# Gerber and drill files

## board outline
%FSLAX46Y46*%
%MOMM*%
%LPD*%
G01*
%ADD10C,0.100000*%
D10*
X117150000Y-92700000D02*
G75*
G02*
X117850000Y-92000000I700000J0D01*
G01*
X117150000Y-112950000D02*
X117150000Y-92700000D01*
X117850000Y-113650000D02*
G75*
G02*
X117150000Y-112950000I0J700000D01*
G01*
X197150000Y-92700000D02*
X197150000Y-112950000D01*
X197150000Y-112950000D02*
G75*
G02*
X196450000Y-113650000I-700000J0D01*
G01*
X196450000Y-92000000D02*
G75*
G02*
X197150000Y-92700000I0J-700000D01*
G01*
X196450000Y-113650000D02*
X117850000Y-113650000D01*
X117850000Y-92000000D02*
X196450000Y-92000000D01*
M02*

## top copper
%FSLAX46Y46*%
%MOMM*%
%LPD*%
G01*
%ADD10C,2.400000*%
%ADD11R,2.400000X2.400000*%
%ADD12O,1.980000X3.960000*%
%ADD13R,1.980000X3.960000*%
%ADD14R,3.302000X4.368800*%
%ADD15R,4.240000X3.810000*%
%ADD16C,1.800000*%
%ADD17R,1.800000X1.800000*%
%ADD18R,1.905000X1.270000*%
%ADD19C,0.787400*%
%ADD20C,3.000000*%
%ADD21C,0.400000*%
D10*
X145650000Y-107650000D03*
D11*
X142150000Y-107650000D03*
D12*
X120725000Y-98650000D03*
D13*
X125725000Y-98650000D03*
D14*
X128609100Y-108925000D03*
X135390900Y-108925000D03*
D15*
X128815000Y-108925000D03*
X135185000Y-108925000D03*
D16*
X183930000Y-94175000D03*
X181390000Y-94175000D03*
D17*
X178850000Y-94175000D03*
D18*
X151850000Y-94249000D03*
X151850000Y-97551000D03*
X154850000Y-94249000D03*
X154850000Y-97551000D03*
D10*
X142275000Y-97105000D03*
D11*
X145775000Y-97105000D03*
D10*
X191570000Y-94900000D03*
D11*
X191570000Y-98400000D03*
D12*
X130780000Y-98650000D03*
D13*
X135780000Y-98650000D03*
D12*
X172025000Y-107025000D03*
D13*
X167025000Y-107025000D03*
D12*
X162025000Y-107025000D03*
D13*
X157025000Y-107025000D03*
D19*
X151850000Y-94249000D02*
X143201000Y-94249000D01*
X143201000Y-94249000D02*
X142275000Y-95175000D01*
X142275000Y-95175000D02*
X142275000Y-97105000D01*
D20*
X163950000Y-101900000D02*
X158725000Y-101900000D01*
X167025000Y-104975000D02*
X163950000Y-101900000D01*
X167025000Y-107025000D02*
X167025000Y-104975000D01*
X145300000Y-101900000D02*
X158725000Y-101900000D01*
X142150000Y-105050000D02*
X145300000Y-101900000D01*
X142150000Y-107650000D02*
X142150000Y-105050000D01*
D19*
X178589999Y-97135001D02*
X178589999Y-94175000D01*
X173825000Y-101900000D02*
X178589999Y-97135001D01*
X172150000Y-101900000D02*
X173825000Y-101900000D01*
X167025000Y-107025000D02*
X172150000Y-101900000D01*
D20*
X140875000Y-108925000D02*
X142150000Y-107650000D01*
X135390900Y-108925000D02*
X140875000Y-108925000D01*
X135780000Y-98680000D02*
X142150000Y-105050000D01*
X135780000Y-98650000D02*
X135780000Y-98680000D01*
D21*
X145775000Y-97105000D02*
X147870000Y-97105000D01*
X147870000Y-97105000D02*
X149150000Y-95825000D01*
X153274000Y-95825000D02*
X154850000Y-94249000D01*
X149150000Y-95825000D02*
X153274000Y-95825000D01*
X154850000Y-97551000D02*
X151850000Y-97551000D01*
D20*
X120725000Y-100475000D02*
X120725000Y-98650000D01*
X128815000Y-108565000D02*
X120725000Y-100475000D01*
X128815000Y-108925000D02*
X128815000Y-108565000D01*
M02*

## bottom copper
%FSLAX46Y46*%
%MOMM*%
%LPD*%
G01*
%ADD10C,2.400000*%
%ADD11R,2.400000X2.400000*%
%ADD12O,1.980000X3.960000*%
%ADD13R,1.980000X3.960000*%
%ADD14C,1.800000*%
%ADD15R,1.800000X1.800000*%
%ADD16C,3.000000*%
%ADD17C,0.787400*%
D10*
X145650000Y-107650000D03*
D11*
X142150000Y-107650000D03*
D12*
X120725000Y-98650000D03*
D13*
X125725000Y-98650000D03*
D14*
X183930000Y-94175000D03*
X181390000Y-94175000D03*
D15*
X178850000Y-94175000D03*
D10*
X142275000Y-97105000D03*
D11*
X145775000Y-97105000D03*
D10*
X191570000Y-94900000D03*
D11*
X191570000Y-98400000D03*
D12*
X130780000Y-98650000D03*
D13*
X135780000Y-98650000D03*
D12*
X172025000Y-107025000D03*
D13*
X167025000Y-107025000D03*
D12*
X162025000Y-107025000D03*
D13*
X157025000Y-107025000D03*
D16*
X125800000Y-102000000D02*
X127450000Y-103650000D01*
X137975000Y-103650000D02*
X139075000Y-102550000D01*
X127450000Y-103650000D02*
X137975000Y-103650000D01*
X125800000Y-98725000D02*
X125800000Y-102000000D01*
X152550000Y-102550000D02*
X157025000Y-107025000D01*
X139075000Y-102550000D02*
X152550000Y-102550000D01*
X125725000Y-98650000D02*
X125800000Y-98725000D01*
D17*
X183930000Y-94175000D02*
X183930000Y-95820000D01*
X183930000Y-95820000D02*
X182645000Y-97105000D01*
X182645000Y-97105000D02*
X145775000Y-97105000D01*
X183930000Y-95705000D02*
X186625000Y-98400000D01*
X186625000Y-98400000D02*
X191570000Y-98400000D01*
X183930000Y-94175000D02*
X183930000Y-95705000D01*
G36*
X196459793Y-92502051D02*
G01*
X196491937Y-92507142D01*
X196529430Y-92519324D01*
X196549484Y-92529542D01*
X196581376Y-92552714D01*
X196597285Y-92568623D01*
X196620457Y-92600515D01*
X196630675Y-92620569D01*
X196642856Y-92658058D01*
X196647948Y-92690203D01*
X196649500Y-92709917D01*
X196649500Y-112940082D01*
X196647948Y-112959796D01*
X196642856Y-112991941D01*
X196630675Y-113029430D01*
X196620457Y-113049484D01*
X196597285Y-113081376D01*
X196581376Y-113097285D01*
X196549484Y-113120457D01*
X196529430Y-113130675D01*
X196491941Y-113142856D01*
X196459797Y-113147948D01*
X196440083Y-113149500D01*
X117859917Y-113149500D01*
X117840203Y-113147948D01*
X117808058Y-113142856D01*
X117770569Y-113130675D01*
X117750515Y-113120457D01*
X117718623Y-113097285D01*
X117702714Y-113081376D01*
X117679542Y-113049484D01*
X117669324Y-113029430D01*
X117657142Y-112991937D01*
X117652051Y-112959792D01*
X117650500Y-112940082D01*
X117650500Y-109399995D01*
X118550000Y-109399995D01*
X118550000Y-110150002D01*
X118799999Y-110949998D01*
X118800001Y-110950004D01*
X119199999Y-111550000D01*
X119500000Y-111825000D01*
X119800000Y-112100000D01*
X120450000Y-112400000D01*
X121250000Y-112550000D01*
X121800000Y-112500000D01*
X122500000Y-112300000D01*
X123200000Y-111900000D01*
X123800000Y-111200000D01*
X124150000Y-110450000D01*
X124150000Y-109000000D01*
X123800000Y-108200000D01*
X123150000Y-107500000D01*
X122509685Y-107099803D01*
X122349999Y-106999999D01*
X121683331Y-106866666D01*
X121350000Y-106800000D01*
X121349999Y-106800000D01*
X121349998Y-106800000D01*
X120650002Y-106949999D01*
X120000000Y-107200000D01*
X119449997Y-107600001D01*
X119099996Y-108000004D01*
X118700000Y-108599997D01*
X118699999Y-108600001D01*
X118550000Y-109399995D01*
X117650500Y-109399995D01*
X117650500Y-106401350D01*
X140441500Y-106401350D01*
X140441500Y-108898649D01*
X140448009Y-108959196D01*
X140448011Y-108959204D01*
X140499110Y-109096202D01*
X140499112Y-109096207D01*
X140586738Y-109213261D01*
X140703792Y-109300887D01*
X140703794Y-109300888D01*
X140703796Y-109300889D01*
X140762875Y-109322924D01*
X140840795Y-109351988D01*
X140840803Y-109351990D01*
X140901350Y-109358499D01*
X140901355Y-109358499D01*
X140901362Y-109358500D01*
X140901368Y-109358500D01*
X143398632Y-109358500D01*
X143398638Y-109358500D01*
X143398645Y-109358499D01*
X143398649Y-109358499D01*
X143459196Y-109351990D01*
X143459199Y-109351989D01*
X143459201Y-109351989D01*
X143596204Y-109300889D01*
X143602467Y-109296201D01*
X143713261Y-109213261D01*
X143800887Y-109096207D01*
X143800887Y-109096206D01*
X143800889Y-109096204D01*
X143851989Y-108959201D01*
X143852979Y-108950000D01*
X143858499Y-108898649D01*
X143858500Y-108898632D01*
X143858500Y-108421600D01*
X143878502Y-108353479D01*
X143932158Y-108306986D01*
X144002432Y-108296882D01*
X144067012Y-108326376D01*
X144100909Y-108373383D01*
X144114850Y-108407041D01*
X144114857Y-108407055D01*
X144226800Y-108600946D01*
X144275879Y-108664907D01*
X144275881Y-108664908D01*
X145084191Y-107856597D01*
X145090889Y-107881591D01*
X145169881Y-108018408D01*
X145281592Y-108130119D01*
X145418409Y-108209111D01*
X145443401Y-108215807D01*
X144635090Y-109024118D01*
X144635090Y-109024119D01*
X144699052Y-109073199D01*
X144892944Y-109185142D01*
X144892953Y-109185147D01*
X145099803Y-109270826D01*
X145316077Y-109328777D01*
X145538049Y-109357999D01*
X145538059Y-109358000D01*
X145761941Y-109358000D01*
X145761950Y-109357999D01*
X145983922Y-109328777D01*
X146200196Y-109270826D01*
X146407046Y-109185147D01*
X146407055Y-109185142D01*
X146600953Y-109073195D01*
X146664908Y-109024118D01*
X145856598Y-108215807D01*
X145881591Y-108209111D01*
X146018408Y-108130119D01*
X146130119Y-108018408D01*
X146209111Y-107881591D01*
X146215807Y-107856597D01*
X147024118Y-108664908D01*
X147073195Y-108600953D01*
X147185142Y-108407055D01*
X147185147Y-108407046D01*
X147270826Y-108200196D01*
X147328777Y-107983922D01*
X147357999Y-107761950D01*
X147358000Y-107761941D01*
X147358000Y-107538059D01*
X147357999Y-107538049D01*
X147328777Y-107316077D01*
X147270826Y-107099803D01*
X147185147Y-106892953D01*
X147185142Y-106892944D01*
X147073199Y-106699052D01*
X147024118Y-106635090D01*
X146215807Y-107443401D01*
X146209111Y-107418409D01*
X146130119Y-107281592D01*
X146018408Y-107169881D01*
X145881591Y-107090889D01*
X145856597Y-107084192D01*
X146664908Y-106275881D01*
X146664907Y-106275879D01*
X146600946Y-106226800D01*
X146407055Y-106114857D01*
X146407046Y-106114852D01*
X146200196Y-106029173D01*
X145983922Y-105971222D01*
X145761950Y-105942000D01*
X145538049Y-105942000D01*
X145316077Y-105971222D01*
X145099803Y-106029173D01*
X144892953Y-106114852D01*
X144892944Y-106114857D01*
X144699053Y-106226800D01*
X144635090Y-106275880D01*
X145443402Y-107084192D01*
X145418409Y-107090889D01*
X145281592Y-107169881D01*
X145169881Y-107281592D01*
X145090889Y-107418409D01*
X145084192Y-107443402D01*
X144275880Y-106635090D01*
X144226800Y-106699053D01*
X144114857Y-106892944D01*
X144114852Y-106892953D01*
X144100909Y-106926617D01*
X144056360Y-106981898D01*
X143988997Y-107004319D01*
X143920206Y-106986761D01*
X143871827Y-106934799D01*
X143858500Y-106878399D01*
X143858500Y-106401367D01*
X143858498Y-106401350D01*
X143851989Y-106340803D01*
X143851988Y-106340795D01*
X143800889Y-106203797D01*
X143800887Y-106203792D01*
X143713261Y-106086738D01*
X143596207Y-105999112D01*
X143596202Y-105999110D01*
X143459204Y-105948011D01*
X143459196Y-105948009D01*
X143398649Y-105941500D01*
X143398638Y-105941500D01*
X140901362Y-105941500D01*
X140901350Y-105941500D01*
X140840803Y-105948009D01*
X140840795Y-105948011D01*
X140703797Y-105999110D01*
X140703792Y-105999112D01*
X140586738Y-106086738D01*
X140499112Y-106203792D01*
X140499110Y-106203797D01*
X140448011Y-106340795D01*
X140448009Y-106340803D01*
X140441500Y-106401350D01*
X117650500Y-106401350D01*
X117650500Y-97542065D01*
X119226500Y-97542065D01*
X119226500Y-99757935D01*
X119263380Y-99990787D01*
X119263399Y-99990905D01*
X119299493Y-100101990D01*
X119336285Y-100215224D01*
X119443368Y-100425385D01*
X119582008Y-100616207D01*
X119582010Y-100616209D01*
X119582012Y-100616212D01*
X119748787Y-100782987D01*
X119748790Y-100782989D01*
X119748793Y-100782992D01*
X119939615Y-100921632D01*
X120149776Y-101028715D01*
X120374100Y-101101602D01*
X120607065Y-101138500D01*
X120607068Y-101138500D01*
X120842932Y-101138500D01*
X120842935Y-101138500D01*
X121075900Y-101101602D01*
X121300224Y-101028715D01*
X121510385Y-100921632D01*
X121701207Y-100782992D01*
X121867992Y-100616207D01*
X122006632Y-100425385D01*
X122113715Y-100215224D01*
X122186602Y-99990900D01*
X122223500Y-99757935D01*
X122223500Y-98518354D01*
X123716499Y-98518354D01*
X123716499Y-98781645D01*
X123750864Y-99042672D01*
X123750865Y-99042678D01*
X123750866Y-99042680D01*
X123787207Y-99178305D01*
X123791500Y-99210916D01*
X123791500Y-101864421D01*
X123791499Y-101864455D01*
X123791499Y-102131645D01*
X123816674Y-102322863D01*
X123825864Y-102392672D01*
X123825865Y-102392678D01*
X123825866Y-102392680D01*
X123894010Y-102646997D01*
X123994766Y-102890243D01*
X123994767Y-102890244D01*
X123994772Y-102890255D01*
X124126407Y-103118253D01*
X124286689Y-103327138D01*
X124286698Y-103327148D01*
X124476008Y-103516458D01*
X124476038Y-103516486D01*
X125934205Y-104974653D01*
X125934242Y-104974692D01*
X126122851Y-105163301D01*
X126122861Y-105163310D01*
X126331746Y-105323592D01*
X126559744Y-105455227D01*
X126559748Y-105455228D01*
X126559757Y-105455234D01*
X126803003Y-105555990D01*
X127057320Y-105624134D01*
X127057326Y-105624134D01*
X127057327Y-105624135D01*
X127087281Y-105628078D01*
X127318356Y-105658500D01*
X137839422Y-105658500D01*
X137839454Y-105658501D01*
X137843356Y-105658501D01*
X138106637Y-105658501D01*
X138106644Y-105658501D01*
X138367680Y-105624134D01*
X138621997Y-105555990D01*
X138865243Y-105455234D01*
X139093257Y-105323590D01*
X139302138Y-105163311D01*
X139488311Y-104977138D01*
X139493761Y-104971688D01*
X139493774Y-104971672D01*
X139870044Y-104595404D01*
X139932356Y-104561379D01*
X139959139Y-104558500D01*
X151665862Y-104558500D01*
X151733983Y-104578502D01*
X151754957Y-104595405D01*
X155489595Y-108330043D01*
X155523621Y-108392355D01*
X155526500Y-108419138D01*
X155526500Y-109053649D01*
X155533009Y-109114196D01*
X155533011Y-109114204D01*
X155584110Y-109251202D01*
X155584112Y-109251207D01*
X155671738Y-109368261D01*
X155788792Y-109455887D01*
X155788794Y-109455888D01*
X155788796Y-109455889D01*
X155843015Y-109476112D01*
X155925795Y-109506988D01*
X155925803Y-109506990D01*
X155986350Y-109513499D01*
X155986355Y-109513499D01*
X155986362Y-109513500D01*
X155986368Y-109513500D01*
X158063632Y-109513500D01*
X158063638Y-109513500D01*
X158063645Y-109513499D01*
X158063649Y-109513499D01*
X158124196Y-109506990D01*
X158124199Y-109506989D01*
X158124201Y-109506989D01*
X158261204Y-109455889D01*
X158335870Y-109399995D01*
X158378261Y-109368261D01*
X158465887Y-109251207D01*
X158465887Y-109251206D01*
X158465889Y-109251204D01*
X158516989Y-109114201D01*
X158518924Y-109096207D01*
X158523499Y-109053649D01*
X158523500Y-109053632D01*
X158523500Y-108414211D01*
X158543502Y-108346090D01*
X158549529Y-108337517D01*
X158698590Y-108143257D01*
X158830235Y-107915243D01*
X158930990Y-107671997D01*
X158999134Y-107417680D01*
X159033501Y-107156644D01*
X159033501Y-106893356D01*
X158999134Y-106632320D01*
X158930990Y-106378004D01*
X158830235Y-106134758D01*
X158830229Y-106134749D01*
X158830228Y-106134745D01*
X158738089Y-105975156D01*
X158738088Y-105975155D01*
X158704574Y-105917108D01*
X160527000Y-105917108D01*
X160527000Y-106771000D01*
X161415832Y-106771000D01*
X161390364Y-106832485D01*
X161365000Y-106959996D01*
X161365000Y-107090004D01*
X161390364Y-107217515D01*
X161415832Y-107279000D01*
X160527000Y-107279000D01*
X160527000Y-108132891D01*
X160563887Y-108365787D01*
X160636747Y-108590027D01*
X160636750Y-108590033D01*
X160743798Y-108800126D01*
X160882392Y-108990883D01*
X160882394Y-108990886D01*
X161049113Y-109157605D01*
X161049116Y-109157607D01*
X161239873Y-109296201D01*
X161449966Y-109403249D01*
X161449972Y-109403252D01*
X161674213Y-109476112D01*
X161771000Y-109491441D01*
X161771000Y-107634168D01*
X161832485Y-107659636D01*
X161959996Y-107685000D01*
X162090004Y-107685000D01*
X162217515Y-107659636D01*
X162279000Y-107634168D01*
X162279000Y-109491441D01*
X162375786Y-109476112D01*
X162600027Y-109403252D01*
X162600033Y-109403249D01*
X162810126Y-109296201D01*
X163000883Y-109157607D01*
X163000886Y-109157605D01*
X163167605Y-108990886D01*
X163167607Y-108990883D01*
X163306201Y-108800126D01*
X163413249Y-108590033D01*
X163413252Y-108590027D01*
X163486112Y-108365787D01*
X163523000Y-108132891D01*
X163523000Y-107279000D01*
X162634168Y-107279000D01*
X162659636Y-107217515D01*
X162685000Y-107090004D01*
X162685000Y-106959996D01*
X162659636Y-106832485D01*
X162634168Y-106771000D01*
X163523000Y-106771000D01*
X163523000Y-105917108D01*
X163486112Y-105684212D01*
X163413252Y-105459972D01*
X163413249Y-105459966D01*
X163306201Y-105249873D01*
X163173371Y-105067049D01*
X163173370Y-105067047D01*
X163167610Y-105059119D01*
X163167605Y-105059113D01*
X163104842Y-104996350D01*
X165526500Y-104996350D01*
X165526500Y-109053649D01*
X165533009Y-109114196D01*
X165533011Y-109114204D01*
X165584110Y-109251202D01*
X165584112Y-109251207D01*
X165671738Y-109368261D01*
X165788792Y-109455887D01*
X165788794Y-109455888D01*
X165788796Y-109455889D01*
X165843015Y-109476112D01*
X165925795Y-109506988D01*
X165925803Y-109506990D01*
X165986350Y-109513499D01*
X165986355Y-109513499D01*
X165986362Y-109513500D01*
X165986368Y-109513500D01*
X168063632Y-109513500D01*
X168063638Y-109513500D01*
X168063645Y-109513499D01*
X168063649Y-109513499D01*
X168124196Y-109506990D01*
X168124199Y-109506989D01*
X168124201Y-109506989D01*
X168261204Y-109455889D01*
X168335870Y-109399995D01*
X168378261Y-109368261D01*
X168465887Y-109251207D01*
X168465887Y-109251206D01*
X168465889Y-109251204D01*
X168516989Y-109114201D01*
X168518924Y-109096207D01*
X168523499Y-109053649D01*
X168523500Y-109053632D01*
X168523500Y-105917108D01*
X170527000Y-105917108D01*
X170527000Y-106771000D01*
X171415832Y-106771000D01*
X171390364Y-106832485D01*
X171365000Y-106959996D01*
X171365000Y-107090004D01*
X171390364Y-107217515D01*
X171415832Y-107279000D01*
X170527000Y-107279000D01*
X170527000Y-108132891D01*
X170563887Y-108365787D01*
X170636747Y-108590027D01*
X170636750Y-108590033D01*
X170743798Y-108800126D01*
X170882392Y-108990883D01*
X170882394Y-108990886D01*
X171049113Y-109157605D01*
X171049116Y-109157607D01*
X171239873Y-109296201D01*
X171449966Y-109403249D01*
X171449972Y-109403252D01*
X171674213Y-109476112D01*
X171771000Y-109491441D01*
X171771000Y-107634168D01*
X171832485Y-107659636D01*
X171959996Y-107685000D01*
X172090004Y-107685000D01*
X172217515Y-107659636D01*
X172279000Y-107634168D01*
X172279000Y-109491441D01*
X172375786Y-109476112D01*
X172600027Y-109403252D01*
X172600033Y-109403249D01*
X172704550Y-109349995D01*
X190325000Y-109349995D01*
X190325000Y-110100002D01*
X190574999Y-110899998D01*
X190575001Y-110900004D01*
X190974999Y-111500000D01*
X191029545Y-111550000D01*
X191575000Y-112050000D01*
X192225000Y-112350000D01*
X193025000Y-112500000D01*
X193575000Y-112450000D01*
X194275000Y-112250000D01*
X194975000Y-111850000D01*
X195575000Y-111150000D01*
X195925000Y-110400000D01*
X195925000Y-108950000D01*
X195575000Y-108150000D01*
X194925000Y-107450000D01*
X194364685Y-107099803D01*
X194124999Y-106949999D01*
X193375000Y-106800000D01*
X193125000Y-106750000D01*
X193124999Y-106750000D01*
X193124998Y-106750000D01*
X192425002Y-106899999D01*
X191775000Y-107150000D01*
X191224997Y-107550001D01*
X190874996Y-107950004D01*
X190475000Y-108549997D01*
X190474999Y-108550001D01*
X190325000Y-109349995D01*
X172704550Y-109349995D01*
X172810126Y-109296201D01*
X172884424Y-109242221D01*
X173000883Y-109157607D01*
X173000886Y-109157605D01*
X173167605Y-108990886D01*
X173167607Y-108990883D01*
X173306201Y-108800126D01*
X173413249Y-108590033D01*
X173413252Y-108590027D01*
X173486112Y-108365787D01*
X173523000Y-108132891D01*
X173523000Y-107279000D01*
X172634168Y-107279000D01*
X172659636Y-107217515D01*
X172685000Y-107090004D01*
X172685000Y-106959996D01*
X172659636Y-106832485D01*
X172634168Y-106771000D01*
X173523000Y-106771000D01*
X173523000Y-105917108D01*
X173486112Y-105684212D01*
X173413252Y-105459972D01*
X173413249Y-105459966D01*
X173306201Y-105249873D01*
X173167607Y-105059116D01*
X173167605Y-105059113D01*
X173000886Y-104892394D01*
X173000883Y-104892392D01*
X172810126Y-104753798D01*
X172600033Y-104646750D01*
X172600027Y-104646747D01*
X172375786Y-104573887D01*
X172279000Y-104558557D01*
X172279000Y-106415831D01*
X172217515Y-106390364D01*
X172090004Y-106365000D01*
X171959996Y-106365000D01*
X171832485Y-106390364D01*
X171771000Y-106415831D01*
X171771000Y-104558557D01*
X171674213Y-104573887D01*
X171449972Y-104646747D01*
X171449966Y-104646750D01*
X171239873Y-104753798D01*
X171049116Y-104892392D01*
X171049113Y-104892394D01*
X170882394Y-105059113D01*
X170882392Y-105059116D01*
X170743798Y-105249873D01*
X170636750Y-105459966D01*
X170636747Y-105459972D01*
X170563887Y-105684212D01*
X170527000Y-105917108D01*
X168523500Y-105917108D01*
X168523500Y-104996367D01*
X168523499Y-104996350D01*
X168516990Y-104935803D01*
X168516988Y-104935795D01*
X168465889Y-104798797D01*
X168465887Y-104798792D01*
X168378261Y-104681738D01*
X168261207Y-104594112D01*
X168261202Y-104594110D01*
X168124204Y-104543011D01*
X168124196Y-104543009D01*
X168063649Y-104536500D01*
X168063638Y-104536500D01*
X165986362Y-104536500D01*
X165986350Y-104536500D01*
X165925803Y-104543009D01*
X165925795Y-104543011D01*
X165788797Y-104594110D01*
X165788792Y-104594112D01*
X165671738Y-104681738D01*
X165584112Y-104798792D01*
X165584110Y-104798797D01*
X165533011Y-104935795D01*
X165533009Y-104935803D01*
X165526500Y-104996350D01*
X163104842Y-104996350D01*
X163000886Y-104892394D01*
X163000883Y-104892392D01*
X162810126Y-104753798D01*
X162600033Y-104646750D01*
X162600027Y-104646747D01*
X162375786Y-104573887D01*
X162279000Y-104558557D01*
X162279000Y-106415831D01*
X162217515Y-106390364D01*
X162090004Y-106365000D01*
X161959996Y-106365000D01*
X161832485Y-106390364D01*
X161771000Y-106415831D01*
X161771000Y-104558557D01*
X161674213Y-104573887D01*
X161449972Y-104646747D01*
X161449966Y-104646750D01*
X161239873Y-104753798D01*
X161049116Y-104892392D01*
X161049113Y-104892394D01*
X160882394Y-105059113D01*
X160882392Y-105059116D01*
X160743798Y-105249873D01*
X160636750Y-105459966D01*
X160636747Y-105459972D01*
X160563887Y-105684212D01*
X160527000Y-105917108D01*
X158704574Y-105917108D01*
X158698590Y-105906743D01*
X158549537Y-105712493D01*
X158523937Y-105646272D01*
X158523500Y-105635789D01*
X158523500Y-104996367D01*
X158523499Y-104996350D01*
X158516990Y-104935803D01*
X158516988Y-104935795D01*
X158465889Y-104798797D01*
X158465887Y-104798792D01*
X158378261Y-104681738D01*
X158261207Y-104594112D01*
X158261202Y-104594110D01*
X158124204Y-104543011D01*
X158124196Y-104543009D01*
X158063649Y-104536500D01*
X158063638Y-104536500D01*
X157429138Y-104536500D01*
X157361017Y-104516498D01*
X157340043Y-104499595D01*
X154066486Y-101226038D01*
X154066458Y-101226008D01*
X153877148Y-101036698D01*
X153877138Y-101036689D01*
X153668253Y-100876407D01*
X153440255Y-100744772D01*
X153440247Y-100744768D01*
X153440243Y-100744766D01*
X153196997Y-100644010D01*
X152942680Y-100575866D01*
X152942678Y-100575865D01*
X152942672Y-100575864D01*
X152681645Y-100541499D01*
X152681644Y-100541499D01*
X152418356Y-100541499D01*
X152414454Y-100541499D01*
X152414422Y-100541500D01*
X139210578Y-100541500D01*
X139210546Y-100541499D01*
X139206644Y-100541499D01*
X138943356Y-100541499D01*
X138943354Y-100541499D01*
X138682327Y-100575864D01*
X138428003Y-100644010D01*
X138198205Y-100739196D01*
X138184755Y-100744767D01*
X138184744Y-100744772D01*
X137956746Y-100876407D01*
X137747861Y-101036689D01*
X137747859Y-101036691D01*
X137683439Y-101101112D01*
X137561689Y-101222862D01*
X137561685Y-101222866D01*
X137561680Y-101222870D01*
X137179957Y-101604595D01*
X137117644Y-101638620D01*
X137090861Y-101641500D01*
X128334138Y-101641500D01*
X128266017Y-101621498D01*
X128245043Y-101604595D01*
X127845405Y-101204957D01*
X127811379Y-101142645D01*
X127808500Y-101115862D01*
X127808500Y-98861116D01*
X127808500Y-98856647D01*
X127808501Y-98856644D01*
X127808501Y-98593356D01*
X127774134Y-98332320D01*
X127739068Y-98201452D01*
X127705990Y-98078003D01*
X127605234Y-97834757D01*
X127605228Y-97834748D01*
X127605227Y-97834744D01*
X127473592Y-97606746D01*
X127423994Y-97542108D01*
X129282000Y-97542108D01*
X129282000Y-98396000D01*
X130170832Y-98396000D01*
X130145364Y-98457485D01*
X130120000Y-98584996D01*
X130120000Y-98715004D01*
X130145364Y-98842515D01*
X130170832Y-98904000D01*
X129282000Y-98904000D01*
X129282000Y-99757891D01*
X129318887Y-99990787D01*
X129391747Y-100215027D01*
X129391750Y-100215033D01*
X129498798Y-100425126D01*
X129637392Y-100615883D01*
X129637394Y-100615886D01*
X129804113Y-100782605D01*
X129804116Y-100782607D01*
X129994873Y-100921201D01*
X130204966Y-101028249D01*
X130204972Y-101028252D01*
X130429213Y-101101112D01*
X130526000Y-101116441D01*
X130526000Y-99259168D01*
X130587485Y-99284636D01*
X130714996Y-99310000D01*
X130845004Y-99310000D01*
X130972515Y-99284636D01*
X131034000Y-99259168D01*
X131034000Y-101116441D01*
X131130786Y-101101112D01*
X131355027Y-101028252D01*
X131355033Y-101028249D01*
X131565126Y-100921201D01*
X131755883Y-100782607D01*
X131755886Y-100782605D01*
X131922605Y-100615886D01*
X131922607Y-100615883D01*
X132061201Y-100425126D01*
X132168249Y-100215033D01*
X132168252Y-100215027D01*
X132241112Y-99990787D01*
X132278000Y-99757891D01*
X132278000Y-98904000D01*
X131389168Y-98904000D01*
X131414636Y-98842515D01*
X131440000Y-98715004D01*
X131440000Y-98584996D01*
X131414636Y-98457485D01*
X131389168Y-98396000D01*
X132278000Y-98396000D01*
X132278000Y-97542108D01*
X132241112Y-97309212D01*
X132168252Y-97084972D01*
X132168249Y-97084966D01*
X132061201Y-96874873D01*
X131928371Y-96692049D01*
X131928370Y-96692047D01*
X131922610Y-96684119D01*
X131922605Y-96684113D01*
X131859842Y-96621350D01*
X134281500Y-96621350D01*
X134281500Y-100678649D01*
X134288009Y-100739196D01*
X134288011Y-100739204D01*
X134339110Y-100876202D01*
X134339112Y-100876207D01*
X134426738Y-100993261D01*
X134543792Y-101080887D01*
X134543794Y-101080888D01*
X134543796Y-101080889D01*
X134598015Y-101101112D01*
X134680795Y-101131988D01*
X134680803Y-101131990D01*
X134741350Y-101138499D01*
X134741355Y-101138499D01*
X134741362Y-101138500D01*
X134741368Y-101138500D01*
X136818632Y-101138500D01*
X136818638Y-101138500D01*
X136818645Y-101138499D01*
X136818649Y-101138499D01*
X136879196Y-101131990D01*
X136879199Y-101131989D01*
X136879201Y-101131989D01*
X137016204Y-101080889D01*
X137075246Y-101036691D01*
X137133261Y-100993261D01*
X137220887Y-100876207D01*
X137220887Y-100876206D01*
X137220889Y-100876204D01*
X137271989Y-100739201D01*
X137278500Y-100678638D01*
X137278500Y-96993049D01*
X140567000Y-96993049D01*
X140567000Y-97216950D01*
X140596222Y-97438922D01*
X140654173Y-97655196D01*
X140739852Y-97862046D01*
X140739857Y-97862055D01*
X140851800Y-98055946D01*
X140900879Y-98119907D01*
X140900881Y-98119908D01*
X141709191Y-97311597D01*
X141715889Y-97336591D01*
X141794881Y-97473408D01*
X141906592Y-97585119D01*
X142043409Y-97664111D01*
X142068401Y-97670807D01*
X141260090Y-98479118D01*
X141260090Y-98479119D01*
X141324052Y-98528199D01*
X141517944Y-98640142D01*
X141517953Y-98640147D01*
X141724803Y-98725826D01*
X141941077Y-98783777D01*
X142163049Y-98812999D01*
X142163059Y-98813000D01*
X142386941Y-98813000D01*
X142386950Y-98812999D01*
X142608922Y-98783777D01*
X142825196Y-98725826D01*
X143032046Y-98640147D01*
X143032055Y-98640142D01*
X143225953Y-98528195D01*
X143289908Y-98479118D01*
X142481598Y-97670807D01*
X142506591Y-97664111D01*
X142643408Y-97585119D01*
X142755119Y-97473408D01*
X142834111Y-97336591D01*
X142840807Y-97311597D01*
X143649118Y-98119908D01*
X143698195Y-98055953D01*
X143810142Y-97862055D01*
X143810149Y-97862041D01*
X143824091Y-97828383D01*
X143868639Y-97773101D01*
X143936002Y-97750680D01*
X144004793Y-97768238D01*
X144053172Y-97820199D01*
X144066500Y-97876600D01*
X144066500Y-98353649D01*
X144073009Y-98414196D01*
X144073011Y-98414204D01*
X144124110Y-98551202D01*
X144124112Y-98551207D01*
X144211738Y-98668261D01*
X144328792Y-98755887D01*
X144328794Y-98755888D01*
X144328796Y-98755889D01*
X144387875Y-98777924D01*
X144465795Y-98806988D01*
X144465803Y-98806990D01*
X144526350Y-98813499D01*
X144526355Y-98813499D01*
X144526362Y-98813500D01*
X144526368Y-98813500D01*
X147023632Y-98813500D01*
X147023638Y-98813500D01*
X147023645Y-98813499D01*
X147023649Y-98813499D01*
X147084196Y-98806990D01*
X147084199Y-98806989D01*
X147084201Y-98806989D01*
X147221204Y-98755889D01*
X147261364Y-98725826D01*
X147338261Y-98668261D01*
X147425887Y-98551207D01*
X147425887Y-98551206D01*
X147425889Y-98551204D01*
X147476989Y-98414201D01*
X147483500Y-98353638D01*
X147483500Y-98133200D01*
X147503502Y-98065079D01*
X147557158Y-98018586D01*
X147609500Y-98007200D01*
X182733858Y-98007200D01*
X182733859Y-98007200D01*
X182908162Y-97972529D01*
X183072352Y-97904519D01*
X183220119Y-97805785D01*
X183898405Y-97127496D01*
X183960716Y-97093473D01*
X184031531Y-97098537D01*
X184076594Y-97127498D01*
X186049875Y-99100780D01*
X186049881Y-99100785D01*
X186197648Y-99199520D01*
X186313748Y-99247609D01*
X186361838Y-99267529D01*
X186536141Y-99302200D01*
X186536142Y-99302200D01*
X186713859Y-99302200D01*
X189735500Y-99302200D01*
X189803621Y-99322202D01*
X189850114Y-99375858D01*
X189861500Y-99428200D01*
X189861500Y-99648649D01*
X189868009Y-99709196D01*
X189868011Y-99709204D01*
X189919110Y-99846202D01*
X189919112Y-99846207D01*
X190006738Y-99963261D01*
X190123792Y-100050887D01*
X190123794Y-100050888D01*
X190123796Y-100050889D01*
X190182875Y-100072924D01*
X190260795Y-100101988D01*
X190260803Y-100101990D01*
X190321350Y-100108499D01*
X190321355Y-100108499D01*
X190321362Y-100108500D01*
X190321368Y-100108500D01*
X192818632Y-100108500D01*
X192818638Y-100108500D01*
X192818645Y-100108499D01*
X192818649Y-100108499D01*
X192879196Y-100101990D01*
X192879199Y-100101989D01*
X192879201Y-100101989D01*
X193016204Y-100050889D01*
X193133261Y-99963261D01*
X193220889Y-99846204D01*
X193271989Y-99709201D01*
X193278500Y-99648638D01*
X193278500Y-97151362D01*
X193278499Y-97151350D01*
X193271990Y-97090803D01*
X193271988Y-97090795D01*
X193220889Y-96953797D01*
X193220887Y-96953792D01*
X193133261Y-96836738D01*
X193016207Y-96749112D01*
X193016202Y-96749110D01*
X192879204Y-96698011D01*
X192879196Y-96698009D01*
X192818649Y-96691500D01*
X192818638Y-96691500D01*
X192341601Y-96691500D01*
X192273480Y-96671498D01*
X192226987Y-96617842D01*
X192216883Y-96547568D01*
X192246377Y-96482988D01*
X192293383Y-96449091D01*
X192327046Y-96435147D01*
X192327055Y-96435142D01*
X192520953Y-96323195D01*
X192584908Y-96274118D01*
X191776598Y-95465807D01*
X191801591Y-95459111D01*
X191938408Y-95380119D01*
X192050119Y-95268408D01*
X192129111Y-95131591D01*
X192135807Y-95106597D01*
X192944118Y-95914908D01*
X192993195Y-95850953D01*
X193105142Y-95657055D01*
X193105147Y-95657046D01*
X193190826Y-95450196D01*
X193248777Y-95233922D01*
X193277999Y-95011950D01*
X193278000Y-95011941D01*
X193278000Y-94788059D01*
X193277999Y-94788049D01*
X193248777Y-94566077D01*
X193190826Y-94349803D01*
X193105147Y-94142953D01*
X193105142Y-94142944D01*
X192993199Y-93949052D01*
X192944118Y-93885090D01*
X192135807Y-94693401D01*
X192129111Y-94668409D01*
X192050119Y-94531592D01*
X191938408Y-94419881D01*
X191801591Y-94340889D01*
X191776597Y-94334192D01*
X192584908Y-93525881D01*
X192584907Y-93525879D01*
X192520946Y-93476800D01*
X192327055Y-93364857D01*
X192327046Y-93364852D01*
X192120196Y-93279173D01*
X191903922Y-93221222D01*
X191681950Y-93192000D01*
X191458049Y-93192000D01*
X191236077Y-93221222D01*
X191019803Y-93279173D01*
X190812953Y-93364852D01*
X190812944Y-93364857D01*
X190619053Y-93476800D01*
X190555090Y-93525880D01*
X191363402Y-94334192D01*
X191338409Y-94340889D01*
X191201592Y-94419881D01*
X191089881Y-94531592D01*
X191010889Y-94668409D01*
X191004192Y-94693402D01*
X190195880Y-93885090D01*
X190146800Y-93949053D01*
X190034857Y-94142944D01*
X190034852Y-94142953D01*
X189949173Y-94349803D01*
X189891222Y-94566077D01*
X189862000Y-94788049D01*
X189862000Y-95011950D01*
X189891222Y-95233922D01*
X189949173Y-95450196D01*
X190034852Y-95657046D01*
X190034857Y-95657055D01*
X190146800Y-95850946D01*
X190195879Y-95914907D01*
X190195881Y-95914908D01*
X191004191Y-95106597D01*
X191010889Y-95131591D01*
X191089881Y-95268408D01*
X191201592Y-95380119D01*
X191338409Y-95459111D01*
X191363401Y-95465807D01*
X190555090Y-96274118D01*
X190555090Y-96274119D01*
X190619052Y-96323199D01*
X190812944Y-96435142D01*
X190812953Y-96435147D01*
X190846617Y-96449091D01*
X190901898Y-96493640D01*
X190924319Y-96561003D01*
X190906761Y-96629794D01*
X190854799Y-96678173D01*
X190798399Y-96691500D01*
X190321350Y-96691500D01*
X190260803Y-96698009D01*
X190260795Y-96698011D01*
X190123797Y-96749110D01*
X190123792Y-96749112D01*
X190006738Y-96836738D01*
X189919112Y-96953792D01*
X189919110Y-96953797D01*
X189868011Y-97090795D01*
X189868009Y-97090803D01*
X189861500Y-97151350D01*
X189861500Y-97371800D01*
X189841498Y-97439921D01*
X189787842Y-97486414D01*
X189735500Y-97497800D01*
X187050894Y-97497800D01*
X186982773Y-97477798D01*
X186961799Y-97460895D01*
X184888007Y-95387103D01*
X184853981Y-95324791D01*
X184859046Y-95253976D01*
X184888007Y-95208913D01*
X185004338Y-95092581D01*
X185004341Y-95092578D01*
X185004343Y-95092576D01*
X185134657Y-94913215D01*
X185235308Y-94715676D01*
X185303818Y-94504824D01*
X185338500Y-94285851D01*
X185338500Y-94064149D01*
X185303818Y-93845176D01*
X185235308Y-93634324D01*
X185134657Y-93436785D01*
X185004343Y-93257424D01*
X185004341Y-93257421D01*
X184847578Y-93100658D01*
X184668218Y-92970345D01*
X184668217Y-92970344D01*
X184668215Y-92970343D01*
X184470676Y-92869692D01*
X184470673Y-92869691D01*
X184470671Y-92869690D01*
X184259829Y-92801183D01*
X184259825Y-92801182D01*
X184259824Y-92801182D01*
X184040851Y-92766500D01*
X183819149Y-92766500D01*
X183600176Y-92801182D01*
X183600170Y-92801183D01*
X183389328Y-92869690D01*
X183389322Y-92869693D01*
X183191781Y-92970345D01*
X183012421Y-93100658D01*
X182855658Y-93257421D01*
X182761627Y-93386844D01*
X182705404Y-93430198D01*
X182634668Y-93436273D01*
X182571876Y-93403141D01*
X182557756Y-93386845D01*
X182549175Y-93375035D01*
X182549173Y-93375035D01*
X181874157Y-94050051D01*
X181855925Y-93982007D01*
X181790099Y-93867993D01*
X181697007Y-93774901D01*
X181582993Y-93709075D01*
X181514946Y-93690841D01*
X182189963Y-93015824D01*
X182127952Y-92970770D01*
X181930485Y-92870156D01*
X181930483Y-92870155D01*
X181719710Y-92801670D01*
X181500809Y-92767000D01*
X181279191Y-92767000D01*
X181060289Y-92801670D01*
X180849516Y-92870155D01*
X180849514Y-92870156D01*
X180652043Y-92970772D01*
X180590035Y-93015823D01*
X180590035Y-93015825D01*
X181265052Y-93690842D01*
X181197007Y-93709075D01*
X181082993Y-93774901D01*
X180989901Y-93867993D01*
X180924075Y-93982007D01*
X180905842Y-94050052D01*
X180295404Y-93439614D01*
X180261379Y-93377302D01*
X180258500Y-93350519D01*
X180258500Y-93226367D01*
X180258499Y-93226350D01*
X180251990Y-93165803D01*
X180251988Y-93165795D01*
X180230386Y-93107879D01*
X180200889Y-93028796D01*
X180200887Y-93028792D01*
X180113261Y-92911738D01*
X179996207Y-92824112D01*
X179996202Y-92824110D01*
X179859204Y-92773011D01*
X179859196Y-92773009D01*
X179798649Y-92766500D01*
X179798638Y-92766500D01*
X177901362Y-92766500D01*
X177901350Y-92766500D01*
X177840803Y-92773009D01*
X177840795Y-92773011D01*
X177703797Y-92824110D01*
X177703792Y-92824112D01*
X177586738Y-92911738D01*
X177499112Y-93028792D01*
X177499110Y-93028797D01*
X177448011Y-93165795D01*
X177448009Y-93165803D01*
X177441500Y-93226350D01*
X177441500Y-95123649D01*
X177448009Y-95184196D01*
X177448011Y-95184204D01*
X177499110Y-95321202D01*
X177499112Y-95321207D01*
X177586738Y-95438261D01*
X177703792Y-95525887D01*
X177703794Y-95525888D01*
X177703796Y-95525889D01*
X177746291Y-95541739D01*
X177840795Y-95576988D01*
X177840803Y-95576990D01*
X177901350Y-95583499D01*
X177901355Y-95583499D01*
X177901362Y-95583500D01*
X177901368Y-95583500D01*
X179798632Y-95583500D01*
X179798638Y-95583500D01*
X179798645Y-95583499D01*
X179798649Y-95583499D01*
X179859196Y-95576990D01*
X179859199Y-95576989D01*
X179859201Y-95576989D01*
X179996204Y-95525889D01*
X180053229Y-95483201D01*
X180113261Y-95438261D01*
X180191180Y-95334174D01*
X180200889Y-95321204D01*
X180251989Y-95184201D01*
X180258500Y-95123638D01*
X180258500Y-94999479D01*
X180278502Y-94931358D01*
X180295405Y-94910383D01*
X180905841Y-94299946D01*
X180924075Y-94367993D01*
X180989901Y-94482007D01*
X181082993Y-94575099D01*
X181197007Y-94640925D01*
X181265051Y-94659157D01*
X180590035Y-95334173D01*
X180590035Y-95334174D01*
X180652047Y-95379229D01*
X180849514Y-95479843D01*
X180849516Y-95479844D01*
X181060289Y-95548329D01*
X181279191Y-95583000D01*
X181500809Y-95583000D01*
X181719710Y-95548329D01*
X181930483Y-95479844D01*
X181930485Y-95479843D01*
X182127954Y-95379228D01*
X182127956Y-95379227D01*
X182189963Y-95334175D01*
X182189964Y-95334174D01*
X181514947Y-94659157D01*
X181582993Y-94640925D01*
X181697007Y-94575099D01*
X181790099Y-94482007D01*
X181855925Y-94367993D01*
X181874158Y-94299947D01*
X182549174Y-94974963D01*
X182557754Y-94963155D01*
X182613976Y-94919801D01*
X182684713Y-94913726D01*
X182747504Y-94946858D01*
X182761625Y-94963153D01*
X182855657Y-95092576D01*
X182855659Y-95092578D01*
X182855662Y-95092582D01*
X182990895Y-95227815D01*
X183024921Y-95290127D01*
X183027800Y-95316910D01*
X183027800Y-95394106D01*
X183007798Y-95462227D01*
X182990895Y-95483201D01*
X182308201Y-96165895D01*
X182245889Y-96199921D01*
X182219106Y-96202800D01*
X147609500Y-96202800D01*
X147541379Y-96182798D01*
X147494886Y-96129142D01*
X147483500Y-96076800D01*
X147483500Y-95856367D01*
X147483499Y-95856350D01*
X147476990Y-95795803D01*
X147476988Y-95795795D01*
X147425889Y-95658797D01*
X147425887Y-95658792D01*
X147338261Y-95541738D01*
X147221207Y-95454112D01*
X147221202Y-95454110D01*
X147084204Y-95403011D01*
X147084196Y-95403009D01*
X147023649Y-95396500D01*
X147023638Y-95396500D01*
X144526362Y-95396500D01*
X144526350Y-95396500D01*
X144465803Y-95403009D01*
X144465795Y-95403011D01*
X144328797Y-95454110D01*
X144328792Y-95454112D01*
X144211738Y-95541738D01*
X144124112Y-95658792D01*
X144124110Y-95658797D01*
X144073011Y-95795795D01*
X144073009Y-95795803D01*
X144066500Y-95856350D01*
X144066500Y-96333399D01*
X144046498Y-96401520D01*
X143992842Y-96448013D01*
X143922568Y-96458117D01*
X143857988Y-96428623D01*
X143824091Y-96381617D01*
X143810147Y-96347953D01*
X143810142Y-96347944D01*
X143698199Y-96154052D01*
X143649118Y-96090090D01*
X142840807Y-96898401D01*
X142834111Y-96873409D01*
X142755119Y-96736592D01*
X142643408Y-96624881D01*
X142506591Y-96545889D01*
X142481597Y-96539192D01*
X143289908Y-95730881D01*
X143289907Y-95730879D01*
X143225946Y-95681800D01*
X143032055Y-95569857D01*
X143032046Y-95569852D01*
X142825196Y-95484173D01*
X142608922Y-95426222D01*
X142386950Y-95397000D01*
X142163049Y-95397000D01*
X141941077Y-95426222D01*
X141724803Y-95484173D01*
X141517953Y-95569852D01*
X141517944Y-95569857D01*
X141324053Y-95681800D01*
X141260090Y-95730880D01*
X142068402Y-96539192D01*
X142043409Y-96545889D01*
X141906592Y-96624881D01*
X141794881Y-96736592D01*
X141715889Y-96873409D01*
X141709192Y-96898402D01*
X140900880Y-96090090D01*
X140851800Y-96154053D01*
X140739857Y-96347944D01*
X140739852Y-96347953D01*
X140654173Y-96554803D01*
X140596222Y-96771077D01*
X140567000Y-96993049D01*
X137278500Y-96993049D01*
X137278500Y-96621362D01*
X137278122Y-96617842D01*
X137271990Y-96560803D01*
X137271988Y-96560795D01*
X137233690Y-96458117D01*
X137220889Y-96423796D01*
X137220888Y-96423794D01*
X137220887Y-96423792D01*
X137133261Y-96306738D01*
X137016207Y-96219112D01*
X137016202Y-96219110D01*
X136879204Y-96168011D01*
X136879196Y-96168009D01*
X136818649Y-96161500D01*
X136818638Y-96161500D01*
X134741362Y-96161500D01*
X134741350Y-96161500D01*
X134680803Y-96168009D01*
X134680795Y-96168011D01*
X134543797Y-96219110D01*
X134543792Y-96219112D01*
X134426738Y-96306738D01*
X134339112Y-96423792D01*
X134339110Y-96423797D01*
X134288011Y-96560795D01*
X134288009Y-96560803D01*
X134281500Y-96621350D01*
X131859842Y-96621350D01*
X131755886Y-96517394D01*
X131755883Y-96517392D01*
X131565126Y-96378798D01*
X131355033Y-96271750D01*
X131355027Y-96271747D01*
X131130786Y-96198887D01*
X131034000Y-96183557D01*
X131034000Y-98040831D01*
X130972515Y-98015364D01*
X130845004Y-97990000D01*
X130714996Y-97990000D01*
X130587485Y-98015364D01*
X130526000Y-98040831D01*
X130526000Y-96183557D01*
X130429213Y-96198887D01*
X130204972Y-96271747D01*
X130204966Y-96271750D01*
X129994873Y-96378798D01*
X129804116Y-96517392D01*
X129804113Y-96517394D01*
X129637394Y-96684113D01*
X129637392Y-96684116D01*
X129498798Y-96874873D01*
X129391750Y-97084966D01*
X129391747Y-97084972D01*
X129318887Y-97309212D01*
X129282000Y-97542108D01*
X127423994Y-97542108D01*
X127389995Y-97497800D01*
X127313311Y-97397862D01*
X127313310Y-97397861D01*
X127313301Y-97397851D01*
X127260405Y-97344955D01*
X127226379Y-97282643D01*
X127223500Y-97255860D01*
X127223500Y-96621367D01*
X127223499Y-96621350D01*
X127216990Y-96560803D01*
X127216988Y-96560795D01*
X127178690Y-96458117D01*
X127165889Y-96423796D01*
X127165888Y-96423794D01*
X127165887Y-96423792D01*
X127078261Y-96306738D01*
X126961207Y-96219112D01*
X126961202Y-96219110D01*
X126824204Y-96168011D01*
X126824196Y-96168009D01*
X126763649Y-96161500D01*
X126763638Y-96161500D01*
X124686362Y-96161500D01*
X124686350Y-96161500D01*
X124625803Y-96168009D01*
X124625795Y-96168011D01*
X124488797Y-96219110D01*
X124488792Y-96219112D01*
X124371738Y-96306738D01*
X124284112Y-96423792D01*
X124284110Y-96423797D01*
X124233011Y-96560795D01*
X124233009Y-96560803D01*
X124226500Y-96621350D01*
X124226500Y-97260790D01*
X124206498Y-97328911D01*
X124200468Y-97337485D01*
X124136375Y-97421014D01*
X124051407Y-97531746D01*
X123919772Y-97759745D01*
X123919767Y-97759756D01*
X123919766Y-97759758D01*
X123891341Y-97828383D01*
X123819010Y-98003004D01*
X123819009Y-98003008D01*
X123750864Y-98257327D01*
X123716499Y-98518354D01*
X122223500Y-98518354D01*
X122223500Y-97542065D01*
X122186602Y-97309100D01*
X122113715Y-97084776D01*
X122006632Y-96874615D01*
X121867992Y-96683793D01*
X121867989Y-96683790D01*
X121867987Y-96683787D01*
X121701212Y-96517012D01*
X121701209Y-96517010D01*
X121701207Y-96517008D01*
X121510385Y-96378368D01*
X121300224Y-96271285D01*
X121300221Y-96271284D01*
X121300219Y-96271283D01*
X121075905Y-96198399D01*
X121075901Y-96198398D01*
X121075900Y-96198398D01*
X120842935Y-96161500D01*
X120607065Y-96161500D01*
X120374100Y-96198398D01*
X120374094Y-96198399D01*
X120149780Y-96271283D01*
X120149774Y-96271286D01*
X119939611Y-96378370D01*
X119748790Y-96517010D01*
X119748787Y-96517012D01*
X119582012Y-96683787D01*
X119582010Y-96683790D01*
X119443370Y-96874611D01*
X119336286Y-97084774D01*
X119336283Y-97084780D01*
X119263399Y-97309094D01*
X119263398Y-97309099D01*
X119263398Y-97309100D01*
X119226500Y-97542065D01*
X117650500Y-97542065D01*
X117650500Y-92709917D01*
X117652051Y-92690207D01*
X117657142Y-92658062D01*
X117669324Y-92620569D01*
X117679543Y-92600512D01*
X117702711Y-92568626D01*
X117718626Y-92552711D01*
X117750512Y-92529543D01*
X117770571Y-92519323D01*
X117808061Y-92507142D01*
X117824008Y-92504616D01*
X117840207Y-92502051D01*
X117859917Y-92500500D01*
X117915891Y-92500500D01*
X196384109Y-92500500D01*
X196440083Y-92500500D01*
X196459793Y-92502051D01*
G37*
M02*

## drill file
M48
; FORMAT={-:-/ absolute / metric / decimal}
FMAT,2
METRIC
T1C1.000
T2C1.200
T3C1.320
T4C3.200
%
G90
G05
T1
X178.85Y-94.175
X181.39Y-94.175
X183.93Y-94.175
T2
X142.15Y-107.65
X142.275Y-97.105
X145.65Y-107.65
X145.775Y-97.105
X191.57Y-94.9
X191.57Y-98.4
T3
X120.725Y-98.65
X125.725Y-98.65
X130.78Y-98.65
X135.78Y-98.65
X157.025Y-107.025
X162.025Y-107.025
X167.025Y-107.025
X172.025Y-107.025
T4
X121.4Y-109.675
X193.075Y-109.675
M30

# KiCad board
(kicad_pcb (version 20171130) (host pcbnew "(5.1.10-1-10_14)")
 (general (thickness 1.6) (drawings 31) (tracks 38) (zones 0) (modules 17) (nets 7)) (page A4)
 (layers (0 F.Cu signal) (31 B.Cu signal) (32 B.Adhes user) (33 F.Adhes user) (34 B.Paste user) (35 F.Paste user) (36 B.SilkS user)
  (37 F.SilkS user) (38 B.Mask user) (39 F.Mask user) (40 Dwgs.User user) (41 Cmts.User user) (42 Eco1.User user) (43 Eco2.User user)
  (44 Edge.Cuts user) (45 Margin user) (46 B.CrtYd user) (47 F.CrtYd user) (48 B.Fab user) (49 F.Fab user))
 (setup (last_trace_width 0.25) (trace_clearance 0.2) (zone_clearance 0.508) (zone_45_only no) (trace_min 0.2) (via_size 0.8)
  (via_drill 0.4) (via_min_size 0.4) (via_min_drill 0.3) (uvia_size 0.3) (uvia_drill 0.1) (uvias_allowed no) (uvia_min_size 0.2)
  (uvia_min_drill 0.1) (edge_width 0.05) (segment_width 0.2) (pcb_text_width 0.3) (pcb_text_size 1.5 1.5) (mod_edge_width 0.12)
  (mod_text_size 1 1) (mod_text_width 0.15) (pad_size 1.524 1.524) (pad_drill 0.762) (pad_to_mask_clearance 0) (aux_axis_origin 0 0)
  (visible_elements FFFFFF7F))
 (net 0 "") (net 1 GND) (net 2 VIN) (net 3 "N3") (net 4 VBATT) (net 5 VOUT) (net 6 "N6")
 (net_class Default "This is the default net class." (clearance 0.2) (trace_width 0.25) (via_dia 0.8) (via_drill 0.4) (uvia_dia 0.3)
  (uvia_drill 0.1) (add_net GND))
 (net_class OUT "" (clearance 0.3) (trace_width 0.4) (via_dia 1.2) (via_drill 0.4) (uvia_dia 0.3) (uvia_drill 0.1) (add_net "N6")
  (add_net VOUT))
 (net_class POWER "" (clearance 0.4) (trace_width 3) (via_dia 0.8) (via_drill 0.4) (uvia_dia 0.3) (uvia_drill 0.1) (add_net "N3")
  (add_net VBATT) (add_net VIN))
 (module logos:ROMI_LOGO (layer B.Cu) (at 181.3 104.625 180)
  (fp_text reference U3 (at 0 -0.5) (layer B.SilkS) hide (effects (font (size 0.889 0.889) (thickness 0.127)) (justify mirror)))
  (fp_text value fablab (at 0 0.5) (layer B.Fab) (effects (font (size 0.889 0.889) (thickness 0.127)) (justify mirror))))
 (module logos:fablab (layer F.Cu) (at 170.575 100.075)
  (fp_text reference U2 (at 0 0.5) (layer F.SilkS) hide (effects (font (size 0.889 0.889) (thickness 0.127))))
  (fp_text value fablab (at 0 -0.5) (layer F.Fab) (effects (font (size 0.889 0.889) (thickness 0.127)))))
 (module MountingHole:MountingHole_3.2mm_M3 (layer F.Cu) (at 121.4 109.675)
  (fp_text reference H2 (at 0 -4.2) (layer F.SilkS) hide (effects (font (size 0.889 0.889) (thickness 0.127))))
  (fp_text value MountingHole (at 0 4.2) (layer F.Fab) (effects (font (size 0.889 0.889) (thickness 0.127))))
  (pad 1 np_thru_hole circle (at 0 0) (size 3.2 3.2) (drill 3.2) (layers *.Cu *.Mask)))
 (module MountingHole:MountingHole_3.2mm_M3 (layer F.Cu) (at 193.075 109.675)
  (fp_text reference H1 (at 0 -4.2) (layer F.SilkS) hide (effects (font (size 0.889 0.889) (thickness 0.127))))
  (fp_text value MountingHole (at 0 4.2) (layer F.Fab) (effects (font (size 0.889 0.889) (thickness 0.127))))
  (pad 1 np_thru_hole circle (at 0 0) (size 3.2 3.2) (drill 3.2) (layers *.Cu *.Mask)))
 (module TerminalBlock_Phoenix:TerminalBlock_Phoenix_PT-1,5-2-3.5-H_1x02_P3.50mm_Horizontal (layer F.Cu) (at 142.15 107.65)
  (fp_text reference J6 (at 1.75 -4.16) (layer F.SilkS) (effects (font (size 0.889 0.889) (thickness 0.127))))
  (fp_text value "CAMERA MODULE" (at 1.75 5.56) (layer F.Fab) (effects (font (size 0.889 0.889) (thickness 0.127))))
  (pad 2 thru_hole circle (at 3.5 0) (size 2.4 2.4) (drill 1.2) (layers *.Cu *.Mask) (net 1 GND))
  (pad 1 thru_hole rect (at 0 0) (size 2.4 2.4) (drill 1.2) (layers *.Cu *.Mask) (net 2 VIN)))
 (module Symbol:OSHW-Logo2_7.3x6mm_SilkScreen (layer F.Cu) (at 162.35 95.65)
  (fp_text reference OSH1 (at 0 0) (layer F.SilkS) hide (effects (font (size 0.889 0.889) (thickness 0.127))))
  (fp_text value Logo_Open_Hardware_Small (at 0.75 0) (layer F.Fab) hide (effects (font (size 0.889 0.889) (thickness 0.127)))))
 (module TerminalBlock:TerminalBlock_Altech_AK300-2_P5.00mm (layer F.Cu) (at 125.725 98.65 180)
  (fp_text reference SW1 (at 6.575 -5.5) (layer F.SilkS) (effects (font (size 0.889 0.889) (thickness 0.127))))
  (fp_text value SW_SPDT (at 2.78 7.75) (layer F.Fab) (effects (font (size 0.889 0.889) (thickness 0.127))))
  (pad 2 thru_hole oval (at 5 0 180) (size 1.98 3.96) (drill 1.32) (layers *.Cu *.Mask) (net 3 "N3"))
  (pad 1 thru_hole rect (at 0 0 180) (size 1.98 3.96) (drill 1.32) (layers *.Cu *.Mask) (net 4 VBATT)))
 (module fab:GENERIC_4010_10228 (layer F.Cu) (at 132 108.925 180)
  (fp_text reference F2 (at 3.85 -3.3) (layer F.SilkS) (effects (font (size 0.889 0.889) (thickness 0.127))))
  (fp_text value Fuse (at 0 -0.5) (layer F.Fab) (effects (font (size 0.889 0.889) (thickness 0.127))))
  (pad 2 smd rect (at 3.3909 0 180) (size 3.302 4.3688) (layers F.Cu F.Paste F.Mask) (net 3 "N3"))
  (pad 1 smd rect (at -3.3909 0 180) (size 3.302 4.3688) (layers F.Cu F.Paste F.Mask) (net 2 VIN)))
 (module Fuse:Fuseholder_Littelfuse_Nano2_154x (layer F.Cu) (at 132 108.925 180)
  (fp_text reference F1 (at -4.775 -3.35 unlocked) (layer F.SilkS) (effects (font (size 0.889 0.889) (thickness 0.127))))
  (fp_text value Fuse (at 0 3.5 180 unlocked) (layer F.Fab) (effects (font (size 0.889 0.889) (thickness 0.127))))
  (pad 2 smd rect (at 3.185 0 180) (size 4.24 3.81) (layers F.Cu F.Paste F.Mask) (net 3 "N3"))
  (pad 1 smd rect (at -3.185 0 180) (size 4.24 3.81) (layers F.Cu F.Paste F.Mask) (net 2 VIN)))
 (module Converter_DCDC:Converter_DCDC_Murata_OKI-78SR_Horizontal (layer F.Cu) (at 178.85 94.175)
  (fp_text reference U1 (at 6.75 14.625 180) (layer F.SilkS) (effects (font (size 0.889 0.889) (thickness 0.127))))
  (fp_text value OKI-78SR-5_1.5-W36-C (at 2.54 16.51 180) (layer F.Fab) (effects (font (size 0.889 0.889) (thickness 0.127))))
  (pad 3 thru_hole circle (at 5.08 0 180) (size 1.8 1.8) (drill 1) (layers *.Cu *.Mask) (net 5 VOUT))
  (pad 2 thru_hole circle (at 2.54 0 180) (size 1.8 1.8) (drill 1) (layers *.Cu *.Mask) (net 1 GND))
  (pad 1 thru_hole rect (at 0 0 180) (size 1.8 1.8) (drill 1) (layers *.Cu *.Mask) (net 2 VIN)))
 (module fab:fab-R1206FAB (layer F.Cu) (at 151.85 95.9 90)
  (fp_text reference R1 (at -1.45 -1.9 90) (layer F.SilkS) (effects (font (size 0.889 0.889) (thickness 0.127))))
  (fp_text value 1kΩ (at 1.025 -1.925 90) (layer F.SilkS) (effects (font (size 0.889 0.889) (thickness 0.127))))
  (pad 2 smd rect (at 1.651 0 90) (size 1.27 1.905) (layers F.Cu F.Paste F.Mask) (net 1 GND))
  (pad 1 smd rect (at -1.651 0 90) (size 1.27 1.905) (layers F.Cu F.Paste F.Mask) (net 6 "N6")))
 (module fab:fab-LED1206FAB (layer F.Cu) (at 154.85 95.9 90)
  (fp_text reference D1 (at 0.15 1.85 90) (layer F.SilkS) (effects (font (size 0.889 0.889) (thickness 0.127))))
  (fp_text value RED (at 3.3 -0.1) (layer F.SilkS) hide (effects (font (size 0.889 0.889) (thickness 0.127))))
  (pad 2 smd rect (at 1.651 0 90) (size 1.27 1.905) (layers F.Cu F.Paste F.Mask) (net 5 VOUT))
  (pad 1 smd rect (at -1.651 0 90) (size 1.27 1.905) (layers F.Cu F.Paste F.Mask) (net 6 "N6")))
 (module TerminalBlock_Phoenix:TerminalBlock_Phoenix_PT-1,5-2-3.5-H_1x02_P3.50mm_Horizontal (layer F.Cu) (at 145.775 97.105 180)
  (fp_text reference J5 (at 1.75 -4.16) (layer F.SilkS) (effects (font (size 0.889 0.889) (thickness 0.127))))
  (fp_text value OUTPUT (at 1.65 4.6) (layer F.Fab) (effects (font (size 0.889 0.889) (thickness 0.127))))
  (pad 2 thru_hole circle (at 3.5 0 180) (size 2.4 2.4) (drill 1.2) (layers *.Cu *.Mask) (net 1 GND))
  (pad 1 thru_hole rect (at 0 0 180) (size 2.4 2.4) (drill 1.2) (layers *.Cu *.Mask) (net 5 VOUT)))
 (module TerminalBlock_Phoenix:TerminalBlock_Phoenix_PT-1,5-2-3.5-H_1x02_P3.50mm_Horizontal (layer F.Cu) (at 191.57 98.4 90)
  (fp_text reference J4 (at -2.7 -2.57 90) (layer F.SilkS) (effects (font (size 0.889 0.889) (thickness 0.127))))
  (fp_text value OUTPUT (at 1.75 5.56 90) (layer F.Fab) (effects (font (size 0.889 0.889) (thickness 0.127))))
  (pad 2 thru_hole circle (at 3.5 0 90) (size 2.4 2.4) (drill 1.2) (layers *.Cu *.Mask) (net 1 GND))
  (pad 1 thru_hole rect (at 0 0 90) (size 2.4 2.4) (drill 1.2) (layers *.Cu *.Mask) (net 5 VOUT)))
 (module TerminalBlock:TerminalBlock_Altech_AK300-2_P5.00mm (layer F.Cu) (at 135.78 98.65 180)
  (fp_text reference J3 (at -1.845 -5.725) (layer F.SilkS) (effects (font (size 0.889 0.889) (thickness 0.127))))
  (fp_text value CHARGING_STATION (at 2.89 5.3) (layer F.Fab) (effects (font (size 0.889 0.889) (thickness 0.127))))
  (pad 2 thru_hole oval (at 5 0 180) (size 1.98 3.96) (drill 1.32) (layers *.Cu *.Mask) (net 1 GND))
  (pad 1 thru_hole rect (at 0 0 180) (size 1.98 3.96) (drill 1.32) (layers *.Cu *.Mask) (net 2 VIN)))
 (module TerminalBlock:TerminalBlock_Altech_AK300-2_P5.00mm (layer F.Cu) (at 167.025 107.025)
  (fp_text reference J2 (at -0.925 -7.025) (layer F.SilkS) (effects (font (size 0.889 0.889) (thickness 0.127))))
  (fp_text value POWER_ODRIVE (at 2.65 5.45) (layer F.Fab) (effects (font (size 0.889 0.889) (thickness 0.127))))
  (pad 2 thru_hole oval (at 5 0) (size 1.98 3.96) (drill 1.32) (layers *.Cu *.Mask) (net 1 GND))
  (pad 1 thru_hole rect (at 0 0) (size 1.98 3.96) (drill 1.32) (layers *.Cu *.Mask) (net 2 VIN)))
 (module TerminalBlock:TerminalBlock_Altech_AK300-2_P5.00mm (layer F.Cu) (at 157.025 107.025)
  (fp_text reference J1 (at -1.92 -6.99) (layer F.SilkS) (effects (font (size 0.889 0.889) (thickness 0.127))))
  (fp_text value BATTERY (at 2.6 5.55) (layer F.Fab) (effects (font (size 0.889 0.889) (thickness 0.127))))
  (pad 2 thru_hole oval (at 5 0) (size 1.98 3.96) (drill 1.32) (layers *.Cu *.Mask) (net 1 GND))
  (pad 1 thru_hole rect (at 0 0) (size 1.98 3.96) (drill 1.32) (layers *.Cu *.Mask) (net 4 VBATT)))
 (gr_arc (start 117.85 92.7) (end 117.85 92) (angle -90) (layer Edge.Cuts) (width 0.1))
 (gr_line (start 117.15 112.95) (end 117.15 92.7) (layer Edge.Cuts) (width 0.1))
 (gr_arc (start 117.85 112.95) (end 117.15 112.95) (angle -90) (layer Edge.Cuts) (width 0.1))
 (gr_line (start 197.15 92.7) (end 197.15 112.95) (layer Edge.Cuts) (width 0.1))
 (gr_arc (start 196.45 112.95) (end 196.45 113.65) (angle -90) (layer Edge.Cuts) (width 0.1))
 (gr_arc (start 196.45 92.7) (end 197.15 92.7) (angle -90) (layer Edge.Cuts) (width 0.1))
 (gr_line (start 196.45 113.65) (end 117.85 113.65) (layer Edge.Cuts) (width 0.1))
 (gr_line (start 117.85 92) (end 196.45 92) (layer Edge.Cuts) (width 0.1))
 (segment (start 151.85 94.249) (end 143.201 94.249) (width 0.7874) (layer F.Cu) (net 1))
 (segment (start 143.201 94.249) (end 142.275 95.175) (width 0.7874) (layer F.Cu) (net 1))
 (segment (start 142.275 95.175) (end 142.275 97.105) (width 0.7874) (layer F.Cu) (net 1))
 (segment (start 163.95 101.9) (end 158.725 101.9) (width 3) (layer F.Cu) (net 2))
 (segment (start 167.025 104.975) (end 163.95 101.9) (width 3) (layer F.Cu) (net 2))
 (segment (start 167.025 107.025) (end 167.025 104.975) (width 3) (layer F.Cu) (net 2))
 (segment (start 145.3 101.9) (end 158.725 101.9) (width 3) (layer F.Cu) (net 2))
 (segment (start 142.15 105.05) (end 145.3 101.9) (width 3) (layer F.Cu) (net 2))
 (segment (start 142.15 107.65) (end 142.15 105.05) (width 3) (layer F.Cu) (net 2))
 (segment (start 178.589999 97.135001) (end 178.589999 94.175) (width 0.7874) (layer F.Cu) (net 2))
 (segment (start 173.825 101.9) (end 178.589999 97.135001) (width 0.7874) (layer F.Cu) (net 2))
 (segment (start 172.15 101.9) (end 173.825 101.9) (width 0.7874) (layer F.Cu) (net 2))
 (segment (start 167.025 107.025) (end 172.15 101.9) (width 0.7874) (layer F.Cu) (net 2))
 (segment (start 140.875 108.925) (end 142.15 107.65) (width 3) (layer F.Cu) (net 2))
 (segment (start 135.3909 108.925) (end 140.875 108.925) (width 3) (layer F.Cu) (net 2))
 (segment (start 135.78 98.68) (end 142.15 105.05) (width 3) (layer F.Cu) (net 2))
 (segment (start 135.78 98.65) (end 135.78 98.68) (width 3) (layer F.Cu) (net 2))
 (segment (start 125.8 102) (end 127.45 103.65) (width 3) (layer B.Cu) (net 4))
 (segment (start 137.975 103.65) (end 139.075 102.55) (width 3) (layer B.Cu) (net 4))
 (segment (start 127.45 103.65) (end 137.975 103.65) (width 3) (layer B.Cu) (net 4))
 (segment (start 125.8 98.725) (end 125.8 102) (width 3) (layer B.Cu) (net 4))
 (segment (start 152.55 102.55) (end 157.025 107.025) (width 3) (layer B.Cu) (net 4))
 (segment (start 139.075 102.55) (end 152.55 102.55) (width 3) (layer B.Cu) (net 4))
 (segment (start 125.725 98.65) (end 125.8 98.725) (width 3) (layer B.Cu) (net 4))
 (segment (start 145.775 97.105) (end 147.87 97.105) (width 0.4) (layer F.Cu) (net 5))
 (segment (start 147.87 97.105) (end 149.15 95.825) (width 0.4) (layer F.Cu) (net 5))
 (segment (start 153.274 95.825) (end 154.85 94.249) (width 0.4) (layer F.Cu) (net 5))
 (segment (start 149.15 95.825) (end 153.274 95.825) (width 0.4) (layer F.Cu) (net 5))
 (segment (start 183.93 94.175) (end 183.93 95.82) (width 0.7874) (layer B.Cu) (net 5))
 (segment (start 183.93 95.82) (end 182.645 97.105) (width 0.7874) (layer B.Cu) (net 5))
 (segment (start 182.645 97.105) (end 145.775 97.105) (width 0.7874) (layer B.Cu) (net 5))
 (segment (start 183.93 95.705) (end 186.625 98.4) (width 0.7874) (layer B.Cu) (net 5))
 (segment (start 186.625 98.4) (end 191.57 98.4) (width 0.7874) (layer B.Cu) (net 5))
 (segment (start 183.93 94.175) (end 183.93 95.705) (width 0.7874) (layer B.Cu) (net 5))
 (segment (start 154.85 97.551) (end 151.85 97.551) (width 0.4) (layer F.Cu) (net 6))
 (segment (start 120.725 100.475) (end 120.725 98.65) (width 3) (layer F.Cu) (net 3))
 (segment (start 128.815 108.565) (end 120.725 100.475) (width 3) (layer F.Cu) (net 3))
 (segment (start 128.815 108.925) (end 128.815 108.565) (width 3) (layer F.Cu) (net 3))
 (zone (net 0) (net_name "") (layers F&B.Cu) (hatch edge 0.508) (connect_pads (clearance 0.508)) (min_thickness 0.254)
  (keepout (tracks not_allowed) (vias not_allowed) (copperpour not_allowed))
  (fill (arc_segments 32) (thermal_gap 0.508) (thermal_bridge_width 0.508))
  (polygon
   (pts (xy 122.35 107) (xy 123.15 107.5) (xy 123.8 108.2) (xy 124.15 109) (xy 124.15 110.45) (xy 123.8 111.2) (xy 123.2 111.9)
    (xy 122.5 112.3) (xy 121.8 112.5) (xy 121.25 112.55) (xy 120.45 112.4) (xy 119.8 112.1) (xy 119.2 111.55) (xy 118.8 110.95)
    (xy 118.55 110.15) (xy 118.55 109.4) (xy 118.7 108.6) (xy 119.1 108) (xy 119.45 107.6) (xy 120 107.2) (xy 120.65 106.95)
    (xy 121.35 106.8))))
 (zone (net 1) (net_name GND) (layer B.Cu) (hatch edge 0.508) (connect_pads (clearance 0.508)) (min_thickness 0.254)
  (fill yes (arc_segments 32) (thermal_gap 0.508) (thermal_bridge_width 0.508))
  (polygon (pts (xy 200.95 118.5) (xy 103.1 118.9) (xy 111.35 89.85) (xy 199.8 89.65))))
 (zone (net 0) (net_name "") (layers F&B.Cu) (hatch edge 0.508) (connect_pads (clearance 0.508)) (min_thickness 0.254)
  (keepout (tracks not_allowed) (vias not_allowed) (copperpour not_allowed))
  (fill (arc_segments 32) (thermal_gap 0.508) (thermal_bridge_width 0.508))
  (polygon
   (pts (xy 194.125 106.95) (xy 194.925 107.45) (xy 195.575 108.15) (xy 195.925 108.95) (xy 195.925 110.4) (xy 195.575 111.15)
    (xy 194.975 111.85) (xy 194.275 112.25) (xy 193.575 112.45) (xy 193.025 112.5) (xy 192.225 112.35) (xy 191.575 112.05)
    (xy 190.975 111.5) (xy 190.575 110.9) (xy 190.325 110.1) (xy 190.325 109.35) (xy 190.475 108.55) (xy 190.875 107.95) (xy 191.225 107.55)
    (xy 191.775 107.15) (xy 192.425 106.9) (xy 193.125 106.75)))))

